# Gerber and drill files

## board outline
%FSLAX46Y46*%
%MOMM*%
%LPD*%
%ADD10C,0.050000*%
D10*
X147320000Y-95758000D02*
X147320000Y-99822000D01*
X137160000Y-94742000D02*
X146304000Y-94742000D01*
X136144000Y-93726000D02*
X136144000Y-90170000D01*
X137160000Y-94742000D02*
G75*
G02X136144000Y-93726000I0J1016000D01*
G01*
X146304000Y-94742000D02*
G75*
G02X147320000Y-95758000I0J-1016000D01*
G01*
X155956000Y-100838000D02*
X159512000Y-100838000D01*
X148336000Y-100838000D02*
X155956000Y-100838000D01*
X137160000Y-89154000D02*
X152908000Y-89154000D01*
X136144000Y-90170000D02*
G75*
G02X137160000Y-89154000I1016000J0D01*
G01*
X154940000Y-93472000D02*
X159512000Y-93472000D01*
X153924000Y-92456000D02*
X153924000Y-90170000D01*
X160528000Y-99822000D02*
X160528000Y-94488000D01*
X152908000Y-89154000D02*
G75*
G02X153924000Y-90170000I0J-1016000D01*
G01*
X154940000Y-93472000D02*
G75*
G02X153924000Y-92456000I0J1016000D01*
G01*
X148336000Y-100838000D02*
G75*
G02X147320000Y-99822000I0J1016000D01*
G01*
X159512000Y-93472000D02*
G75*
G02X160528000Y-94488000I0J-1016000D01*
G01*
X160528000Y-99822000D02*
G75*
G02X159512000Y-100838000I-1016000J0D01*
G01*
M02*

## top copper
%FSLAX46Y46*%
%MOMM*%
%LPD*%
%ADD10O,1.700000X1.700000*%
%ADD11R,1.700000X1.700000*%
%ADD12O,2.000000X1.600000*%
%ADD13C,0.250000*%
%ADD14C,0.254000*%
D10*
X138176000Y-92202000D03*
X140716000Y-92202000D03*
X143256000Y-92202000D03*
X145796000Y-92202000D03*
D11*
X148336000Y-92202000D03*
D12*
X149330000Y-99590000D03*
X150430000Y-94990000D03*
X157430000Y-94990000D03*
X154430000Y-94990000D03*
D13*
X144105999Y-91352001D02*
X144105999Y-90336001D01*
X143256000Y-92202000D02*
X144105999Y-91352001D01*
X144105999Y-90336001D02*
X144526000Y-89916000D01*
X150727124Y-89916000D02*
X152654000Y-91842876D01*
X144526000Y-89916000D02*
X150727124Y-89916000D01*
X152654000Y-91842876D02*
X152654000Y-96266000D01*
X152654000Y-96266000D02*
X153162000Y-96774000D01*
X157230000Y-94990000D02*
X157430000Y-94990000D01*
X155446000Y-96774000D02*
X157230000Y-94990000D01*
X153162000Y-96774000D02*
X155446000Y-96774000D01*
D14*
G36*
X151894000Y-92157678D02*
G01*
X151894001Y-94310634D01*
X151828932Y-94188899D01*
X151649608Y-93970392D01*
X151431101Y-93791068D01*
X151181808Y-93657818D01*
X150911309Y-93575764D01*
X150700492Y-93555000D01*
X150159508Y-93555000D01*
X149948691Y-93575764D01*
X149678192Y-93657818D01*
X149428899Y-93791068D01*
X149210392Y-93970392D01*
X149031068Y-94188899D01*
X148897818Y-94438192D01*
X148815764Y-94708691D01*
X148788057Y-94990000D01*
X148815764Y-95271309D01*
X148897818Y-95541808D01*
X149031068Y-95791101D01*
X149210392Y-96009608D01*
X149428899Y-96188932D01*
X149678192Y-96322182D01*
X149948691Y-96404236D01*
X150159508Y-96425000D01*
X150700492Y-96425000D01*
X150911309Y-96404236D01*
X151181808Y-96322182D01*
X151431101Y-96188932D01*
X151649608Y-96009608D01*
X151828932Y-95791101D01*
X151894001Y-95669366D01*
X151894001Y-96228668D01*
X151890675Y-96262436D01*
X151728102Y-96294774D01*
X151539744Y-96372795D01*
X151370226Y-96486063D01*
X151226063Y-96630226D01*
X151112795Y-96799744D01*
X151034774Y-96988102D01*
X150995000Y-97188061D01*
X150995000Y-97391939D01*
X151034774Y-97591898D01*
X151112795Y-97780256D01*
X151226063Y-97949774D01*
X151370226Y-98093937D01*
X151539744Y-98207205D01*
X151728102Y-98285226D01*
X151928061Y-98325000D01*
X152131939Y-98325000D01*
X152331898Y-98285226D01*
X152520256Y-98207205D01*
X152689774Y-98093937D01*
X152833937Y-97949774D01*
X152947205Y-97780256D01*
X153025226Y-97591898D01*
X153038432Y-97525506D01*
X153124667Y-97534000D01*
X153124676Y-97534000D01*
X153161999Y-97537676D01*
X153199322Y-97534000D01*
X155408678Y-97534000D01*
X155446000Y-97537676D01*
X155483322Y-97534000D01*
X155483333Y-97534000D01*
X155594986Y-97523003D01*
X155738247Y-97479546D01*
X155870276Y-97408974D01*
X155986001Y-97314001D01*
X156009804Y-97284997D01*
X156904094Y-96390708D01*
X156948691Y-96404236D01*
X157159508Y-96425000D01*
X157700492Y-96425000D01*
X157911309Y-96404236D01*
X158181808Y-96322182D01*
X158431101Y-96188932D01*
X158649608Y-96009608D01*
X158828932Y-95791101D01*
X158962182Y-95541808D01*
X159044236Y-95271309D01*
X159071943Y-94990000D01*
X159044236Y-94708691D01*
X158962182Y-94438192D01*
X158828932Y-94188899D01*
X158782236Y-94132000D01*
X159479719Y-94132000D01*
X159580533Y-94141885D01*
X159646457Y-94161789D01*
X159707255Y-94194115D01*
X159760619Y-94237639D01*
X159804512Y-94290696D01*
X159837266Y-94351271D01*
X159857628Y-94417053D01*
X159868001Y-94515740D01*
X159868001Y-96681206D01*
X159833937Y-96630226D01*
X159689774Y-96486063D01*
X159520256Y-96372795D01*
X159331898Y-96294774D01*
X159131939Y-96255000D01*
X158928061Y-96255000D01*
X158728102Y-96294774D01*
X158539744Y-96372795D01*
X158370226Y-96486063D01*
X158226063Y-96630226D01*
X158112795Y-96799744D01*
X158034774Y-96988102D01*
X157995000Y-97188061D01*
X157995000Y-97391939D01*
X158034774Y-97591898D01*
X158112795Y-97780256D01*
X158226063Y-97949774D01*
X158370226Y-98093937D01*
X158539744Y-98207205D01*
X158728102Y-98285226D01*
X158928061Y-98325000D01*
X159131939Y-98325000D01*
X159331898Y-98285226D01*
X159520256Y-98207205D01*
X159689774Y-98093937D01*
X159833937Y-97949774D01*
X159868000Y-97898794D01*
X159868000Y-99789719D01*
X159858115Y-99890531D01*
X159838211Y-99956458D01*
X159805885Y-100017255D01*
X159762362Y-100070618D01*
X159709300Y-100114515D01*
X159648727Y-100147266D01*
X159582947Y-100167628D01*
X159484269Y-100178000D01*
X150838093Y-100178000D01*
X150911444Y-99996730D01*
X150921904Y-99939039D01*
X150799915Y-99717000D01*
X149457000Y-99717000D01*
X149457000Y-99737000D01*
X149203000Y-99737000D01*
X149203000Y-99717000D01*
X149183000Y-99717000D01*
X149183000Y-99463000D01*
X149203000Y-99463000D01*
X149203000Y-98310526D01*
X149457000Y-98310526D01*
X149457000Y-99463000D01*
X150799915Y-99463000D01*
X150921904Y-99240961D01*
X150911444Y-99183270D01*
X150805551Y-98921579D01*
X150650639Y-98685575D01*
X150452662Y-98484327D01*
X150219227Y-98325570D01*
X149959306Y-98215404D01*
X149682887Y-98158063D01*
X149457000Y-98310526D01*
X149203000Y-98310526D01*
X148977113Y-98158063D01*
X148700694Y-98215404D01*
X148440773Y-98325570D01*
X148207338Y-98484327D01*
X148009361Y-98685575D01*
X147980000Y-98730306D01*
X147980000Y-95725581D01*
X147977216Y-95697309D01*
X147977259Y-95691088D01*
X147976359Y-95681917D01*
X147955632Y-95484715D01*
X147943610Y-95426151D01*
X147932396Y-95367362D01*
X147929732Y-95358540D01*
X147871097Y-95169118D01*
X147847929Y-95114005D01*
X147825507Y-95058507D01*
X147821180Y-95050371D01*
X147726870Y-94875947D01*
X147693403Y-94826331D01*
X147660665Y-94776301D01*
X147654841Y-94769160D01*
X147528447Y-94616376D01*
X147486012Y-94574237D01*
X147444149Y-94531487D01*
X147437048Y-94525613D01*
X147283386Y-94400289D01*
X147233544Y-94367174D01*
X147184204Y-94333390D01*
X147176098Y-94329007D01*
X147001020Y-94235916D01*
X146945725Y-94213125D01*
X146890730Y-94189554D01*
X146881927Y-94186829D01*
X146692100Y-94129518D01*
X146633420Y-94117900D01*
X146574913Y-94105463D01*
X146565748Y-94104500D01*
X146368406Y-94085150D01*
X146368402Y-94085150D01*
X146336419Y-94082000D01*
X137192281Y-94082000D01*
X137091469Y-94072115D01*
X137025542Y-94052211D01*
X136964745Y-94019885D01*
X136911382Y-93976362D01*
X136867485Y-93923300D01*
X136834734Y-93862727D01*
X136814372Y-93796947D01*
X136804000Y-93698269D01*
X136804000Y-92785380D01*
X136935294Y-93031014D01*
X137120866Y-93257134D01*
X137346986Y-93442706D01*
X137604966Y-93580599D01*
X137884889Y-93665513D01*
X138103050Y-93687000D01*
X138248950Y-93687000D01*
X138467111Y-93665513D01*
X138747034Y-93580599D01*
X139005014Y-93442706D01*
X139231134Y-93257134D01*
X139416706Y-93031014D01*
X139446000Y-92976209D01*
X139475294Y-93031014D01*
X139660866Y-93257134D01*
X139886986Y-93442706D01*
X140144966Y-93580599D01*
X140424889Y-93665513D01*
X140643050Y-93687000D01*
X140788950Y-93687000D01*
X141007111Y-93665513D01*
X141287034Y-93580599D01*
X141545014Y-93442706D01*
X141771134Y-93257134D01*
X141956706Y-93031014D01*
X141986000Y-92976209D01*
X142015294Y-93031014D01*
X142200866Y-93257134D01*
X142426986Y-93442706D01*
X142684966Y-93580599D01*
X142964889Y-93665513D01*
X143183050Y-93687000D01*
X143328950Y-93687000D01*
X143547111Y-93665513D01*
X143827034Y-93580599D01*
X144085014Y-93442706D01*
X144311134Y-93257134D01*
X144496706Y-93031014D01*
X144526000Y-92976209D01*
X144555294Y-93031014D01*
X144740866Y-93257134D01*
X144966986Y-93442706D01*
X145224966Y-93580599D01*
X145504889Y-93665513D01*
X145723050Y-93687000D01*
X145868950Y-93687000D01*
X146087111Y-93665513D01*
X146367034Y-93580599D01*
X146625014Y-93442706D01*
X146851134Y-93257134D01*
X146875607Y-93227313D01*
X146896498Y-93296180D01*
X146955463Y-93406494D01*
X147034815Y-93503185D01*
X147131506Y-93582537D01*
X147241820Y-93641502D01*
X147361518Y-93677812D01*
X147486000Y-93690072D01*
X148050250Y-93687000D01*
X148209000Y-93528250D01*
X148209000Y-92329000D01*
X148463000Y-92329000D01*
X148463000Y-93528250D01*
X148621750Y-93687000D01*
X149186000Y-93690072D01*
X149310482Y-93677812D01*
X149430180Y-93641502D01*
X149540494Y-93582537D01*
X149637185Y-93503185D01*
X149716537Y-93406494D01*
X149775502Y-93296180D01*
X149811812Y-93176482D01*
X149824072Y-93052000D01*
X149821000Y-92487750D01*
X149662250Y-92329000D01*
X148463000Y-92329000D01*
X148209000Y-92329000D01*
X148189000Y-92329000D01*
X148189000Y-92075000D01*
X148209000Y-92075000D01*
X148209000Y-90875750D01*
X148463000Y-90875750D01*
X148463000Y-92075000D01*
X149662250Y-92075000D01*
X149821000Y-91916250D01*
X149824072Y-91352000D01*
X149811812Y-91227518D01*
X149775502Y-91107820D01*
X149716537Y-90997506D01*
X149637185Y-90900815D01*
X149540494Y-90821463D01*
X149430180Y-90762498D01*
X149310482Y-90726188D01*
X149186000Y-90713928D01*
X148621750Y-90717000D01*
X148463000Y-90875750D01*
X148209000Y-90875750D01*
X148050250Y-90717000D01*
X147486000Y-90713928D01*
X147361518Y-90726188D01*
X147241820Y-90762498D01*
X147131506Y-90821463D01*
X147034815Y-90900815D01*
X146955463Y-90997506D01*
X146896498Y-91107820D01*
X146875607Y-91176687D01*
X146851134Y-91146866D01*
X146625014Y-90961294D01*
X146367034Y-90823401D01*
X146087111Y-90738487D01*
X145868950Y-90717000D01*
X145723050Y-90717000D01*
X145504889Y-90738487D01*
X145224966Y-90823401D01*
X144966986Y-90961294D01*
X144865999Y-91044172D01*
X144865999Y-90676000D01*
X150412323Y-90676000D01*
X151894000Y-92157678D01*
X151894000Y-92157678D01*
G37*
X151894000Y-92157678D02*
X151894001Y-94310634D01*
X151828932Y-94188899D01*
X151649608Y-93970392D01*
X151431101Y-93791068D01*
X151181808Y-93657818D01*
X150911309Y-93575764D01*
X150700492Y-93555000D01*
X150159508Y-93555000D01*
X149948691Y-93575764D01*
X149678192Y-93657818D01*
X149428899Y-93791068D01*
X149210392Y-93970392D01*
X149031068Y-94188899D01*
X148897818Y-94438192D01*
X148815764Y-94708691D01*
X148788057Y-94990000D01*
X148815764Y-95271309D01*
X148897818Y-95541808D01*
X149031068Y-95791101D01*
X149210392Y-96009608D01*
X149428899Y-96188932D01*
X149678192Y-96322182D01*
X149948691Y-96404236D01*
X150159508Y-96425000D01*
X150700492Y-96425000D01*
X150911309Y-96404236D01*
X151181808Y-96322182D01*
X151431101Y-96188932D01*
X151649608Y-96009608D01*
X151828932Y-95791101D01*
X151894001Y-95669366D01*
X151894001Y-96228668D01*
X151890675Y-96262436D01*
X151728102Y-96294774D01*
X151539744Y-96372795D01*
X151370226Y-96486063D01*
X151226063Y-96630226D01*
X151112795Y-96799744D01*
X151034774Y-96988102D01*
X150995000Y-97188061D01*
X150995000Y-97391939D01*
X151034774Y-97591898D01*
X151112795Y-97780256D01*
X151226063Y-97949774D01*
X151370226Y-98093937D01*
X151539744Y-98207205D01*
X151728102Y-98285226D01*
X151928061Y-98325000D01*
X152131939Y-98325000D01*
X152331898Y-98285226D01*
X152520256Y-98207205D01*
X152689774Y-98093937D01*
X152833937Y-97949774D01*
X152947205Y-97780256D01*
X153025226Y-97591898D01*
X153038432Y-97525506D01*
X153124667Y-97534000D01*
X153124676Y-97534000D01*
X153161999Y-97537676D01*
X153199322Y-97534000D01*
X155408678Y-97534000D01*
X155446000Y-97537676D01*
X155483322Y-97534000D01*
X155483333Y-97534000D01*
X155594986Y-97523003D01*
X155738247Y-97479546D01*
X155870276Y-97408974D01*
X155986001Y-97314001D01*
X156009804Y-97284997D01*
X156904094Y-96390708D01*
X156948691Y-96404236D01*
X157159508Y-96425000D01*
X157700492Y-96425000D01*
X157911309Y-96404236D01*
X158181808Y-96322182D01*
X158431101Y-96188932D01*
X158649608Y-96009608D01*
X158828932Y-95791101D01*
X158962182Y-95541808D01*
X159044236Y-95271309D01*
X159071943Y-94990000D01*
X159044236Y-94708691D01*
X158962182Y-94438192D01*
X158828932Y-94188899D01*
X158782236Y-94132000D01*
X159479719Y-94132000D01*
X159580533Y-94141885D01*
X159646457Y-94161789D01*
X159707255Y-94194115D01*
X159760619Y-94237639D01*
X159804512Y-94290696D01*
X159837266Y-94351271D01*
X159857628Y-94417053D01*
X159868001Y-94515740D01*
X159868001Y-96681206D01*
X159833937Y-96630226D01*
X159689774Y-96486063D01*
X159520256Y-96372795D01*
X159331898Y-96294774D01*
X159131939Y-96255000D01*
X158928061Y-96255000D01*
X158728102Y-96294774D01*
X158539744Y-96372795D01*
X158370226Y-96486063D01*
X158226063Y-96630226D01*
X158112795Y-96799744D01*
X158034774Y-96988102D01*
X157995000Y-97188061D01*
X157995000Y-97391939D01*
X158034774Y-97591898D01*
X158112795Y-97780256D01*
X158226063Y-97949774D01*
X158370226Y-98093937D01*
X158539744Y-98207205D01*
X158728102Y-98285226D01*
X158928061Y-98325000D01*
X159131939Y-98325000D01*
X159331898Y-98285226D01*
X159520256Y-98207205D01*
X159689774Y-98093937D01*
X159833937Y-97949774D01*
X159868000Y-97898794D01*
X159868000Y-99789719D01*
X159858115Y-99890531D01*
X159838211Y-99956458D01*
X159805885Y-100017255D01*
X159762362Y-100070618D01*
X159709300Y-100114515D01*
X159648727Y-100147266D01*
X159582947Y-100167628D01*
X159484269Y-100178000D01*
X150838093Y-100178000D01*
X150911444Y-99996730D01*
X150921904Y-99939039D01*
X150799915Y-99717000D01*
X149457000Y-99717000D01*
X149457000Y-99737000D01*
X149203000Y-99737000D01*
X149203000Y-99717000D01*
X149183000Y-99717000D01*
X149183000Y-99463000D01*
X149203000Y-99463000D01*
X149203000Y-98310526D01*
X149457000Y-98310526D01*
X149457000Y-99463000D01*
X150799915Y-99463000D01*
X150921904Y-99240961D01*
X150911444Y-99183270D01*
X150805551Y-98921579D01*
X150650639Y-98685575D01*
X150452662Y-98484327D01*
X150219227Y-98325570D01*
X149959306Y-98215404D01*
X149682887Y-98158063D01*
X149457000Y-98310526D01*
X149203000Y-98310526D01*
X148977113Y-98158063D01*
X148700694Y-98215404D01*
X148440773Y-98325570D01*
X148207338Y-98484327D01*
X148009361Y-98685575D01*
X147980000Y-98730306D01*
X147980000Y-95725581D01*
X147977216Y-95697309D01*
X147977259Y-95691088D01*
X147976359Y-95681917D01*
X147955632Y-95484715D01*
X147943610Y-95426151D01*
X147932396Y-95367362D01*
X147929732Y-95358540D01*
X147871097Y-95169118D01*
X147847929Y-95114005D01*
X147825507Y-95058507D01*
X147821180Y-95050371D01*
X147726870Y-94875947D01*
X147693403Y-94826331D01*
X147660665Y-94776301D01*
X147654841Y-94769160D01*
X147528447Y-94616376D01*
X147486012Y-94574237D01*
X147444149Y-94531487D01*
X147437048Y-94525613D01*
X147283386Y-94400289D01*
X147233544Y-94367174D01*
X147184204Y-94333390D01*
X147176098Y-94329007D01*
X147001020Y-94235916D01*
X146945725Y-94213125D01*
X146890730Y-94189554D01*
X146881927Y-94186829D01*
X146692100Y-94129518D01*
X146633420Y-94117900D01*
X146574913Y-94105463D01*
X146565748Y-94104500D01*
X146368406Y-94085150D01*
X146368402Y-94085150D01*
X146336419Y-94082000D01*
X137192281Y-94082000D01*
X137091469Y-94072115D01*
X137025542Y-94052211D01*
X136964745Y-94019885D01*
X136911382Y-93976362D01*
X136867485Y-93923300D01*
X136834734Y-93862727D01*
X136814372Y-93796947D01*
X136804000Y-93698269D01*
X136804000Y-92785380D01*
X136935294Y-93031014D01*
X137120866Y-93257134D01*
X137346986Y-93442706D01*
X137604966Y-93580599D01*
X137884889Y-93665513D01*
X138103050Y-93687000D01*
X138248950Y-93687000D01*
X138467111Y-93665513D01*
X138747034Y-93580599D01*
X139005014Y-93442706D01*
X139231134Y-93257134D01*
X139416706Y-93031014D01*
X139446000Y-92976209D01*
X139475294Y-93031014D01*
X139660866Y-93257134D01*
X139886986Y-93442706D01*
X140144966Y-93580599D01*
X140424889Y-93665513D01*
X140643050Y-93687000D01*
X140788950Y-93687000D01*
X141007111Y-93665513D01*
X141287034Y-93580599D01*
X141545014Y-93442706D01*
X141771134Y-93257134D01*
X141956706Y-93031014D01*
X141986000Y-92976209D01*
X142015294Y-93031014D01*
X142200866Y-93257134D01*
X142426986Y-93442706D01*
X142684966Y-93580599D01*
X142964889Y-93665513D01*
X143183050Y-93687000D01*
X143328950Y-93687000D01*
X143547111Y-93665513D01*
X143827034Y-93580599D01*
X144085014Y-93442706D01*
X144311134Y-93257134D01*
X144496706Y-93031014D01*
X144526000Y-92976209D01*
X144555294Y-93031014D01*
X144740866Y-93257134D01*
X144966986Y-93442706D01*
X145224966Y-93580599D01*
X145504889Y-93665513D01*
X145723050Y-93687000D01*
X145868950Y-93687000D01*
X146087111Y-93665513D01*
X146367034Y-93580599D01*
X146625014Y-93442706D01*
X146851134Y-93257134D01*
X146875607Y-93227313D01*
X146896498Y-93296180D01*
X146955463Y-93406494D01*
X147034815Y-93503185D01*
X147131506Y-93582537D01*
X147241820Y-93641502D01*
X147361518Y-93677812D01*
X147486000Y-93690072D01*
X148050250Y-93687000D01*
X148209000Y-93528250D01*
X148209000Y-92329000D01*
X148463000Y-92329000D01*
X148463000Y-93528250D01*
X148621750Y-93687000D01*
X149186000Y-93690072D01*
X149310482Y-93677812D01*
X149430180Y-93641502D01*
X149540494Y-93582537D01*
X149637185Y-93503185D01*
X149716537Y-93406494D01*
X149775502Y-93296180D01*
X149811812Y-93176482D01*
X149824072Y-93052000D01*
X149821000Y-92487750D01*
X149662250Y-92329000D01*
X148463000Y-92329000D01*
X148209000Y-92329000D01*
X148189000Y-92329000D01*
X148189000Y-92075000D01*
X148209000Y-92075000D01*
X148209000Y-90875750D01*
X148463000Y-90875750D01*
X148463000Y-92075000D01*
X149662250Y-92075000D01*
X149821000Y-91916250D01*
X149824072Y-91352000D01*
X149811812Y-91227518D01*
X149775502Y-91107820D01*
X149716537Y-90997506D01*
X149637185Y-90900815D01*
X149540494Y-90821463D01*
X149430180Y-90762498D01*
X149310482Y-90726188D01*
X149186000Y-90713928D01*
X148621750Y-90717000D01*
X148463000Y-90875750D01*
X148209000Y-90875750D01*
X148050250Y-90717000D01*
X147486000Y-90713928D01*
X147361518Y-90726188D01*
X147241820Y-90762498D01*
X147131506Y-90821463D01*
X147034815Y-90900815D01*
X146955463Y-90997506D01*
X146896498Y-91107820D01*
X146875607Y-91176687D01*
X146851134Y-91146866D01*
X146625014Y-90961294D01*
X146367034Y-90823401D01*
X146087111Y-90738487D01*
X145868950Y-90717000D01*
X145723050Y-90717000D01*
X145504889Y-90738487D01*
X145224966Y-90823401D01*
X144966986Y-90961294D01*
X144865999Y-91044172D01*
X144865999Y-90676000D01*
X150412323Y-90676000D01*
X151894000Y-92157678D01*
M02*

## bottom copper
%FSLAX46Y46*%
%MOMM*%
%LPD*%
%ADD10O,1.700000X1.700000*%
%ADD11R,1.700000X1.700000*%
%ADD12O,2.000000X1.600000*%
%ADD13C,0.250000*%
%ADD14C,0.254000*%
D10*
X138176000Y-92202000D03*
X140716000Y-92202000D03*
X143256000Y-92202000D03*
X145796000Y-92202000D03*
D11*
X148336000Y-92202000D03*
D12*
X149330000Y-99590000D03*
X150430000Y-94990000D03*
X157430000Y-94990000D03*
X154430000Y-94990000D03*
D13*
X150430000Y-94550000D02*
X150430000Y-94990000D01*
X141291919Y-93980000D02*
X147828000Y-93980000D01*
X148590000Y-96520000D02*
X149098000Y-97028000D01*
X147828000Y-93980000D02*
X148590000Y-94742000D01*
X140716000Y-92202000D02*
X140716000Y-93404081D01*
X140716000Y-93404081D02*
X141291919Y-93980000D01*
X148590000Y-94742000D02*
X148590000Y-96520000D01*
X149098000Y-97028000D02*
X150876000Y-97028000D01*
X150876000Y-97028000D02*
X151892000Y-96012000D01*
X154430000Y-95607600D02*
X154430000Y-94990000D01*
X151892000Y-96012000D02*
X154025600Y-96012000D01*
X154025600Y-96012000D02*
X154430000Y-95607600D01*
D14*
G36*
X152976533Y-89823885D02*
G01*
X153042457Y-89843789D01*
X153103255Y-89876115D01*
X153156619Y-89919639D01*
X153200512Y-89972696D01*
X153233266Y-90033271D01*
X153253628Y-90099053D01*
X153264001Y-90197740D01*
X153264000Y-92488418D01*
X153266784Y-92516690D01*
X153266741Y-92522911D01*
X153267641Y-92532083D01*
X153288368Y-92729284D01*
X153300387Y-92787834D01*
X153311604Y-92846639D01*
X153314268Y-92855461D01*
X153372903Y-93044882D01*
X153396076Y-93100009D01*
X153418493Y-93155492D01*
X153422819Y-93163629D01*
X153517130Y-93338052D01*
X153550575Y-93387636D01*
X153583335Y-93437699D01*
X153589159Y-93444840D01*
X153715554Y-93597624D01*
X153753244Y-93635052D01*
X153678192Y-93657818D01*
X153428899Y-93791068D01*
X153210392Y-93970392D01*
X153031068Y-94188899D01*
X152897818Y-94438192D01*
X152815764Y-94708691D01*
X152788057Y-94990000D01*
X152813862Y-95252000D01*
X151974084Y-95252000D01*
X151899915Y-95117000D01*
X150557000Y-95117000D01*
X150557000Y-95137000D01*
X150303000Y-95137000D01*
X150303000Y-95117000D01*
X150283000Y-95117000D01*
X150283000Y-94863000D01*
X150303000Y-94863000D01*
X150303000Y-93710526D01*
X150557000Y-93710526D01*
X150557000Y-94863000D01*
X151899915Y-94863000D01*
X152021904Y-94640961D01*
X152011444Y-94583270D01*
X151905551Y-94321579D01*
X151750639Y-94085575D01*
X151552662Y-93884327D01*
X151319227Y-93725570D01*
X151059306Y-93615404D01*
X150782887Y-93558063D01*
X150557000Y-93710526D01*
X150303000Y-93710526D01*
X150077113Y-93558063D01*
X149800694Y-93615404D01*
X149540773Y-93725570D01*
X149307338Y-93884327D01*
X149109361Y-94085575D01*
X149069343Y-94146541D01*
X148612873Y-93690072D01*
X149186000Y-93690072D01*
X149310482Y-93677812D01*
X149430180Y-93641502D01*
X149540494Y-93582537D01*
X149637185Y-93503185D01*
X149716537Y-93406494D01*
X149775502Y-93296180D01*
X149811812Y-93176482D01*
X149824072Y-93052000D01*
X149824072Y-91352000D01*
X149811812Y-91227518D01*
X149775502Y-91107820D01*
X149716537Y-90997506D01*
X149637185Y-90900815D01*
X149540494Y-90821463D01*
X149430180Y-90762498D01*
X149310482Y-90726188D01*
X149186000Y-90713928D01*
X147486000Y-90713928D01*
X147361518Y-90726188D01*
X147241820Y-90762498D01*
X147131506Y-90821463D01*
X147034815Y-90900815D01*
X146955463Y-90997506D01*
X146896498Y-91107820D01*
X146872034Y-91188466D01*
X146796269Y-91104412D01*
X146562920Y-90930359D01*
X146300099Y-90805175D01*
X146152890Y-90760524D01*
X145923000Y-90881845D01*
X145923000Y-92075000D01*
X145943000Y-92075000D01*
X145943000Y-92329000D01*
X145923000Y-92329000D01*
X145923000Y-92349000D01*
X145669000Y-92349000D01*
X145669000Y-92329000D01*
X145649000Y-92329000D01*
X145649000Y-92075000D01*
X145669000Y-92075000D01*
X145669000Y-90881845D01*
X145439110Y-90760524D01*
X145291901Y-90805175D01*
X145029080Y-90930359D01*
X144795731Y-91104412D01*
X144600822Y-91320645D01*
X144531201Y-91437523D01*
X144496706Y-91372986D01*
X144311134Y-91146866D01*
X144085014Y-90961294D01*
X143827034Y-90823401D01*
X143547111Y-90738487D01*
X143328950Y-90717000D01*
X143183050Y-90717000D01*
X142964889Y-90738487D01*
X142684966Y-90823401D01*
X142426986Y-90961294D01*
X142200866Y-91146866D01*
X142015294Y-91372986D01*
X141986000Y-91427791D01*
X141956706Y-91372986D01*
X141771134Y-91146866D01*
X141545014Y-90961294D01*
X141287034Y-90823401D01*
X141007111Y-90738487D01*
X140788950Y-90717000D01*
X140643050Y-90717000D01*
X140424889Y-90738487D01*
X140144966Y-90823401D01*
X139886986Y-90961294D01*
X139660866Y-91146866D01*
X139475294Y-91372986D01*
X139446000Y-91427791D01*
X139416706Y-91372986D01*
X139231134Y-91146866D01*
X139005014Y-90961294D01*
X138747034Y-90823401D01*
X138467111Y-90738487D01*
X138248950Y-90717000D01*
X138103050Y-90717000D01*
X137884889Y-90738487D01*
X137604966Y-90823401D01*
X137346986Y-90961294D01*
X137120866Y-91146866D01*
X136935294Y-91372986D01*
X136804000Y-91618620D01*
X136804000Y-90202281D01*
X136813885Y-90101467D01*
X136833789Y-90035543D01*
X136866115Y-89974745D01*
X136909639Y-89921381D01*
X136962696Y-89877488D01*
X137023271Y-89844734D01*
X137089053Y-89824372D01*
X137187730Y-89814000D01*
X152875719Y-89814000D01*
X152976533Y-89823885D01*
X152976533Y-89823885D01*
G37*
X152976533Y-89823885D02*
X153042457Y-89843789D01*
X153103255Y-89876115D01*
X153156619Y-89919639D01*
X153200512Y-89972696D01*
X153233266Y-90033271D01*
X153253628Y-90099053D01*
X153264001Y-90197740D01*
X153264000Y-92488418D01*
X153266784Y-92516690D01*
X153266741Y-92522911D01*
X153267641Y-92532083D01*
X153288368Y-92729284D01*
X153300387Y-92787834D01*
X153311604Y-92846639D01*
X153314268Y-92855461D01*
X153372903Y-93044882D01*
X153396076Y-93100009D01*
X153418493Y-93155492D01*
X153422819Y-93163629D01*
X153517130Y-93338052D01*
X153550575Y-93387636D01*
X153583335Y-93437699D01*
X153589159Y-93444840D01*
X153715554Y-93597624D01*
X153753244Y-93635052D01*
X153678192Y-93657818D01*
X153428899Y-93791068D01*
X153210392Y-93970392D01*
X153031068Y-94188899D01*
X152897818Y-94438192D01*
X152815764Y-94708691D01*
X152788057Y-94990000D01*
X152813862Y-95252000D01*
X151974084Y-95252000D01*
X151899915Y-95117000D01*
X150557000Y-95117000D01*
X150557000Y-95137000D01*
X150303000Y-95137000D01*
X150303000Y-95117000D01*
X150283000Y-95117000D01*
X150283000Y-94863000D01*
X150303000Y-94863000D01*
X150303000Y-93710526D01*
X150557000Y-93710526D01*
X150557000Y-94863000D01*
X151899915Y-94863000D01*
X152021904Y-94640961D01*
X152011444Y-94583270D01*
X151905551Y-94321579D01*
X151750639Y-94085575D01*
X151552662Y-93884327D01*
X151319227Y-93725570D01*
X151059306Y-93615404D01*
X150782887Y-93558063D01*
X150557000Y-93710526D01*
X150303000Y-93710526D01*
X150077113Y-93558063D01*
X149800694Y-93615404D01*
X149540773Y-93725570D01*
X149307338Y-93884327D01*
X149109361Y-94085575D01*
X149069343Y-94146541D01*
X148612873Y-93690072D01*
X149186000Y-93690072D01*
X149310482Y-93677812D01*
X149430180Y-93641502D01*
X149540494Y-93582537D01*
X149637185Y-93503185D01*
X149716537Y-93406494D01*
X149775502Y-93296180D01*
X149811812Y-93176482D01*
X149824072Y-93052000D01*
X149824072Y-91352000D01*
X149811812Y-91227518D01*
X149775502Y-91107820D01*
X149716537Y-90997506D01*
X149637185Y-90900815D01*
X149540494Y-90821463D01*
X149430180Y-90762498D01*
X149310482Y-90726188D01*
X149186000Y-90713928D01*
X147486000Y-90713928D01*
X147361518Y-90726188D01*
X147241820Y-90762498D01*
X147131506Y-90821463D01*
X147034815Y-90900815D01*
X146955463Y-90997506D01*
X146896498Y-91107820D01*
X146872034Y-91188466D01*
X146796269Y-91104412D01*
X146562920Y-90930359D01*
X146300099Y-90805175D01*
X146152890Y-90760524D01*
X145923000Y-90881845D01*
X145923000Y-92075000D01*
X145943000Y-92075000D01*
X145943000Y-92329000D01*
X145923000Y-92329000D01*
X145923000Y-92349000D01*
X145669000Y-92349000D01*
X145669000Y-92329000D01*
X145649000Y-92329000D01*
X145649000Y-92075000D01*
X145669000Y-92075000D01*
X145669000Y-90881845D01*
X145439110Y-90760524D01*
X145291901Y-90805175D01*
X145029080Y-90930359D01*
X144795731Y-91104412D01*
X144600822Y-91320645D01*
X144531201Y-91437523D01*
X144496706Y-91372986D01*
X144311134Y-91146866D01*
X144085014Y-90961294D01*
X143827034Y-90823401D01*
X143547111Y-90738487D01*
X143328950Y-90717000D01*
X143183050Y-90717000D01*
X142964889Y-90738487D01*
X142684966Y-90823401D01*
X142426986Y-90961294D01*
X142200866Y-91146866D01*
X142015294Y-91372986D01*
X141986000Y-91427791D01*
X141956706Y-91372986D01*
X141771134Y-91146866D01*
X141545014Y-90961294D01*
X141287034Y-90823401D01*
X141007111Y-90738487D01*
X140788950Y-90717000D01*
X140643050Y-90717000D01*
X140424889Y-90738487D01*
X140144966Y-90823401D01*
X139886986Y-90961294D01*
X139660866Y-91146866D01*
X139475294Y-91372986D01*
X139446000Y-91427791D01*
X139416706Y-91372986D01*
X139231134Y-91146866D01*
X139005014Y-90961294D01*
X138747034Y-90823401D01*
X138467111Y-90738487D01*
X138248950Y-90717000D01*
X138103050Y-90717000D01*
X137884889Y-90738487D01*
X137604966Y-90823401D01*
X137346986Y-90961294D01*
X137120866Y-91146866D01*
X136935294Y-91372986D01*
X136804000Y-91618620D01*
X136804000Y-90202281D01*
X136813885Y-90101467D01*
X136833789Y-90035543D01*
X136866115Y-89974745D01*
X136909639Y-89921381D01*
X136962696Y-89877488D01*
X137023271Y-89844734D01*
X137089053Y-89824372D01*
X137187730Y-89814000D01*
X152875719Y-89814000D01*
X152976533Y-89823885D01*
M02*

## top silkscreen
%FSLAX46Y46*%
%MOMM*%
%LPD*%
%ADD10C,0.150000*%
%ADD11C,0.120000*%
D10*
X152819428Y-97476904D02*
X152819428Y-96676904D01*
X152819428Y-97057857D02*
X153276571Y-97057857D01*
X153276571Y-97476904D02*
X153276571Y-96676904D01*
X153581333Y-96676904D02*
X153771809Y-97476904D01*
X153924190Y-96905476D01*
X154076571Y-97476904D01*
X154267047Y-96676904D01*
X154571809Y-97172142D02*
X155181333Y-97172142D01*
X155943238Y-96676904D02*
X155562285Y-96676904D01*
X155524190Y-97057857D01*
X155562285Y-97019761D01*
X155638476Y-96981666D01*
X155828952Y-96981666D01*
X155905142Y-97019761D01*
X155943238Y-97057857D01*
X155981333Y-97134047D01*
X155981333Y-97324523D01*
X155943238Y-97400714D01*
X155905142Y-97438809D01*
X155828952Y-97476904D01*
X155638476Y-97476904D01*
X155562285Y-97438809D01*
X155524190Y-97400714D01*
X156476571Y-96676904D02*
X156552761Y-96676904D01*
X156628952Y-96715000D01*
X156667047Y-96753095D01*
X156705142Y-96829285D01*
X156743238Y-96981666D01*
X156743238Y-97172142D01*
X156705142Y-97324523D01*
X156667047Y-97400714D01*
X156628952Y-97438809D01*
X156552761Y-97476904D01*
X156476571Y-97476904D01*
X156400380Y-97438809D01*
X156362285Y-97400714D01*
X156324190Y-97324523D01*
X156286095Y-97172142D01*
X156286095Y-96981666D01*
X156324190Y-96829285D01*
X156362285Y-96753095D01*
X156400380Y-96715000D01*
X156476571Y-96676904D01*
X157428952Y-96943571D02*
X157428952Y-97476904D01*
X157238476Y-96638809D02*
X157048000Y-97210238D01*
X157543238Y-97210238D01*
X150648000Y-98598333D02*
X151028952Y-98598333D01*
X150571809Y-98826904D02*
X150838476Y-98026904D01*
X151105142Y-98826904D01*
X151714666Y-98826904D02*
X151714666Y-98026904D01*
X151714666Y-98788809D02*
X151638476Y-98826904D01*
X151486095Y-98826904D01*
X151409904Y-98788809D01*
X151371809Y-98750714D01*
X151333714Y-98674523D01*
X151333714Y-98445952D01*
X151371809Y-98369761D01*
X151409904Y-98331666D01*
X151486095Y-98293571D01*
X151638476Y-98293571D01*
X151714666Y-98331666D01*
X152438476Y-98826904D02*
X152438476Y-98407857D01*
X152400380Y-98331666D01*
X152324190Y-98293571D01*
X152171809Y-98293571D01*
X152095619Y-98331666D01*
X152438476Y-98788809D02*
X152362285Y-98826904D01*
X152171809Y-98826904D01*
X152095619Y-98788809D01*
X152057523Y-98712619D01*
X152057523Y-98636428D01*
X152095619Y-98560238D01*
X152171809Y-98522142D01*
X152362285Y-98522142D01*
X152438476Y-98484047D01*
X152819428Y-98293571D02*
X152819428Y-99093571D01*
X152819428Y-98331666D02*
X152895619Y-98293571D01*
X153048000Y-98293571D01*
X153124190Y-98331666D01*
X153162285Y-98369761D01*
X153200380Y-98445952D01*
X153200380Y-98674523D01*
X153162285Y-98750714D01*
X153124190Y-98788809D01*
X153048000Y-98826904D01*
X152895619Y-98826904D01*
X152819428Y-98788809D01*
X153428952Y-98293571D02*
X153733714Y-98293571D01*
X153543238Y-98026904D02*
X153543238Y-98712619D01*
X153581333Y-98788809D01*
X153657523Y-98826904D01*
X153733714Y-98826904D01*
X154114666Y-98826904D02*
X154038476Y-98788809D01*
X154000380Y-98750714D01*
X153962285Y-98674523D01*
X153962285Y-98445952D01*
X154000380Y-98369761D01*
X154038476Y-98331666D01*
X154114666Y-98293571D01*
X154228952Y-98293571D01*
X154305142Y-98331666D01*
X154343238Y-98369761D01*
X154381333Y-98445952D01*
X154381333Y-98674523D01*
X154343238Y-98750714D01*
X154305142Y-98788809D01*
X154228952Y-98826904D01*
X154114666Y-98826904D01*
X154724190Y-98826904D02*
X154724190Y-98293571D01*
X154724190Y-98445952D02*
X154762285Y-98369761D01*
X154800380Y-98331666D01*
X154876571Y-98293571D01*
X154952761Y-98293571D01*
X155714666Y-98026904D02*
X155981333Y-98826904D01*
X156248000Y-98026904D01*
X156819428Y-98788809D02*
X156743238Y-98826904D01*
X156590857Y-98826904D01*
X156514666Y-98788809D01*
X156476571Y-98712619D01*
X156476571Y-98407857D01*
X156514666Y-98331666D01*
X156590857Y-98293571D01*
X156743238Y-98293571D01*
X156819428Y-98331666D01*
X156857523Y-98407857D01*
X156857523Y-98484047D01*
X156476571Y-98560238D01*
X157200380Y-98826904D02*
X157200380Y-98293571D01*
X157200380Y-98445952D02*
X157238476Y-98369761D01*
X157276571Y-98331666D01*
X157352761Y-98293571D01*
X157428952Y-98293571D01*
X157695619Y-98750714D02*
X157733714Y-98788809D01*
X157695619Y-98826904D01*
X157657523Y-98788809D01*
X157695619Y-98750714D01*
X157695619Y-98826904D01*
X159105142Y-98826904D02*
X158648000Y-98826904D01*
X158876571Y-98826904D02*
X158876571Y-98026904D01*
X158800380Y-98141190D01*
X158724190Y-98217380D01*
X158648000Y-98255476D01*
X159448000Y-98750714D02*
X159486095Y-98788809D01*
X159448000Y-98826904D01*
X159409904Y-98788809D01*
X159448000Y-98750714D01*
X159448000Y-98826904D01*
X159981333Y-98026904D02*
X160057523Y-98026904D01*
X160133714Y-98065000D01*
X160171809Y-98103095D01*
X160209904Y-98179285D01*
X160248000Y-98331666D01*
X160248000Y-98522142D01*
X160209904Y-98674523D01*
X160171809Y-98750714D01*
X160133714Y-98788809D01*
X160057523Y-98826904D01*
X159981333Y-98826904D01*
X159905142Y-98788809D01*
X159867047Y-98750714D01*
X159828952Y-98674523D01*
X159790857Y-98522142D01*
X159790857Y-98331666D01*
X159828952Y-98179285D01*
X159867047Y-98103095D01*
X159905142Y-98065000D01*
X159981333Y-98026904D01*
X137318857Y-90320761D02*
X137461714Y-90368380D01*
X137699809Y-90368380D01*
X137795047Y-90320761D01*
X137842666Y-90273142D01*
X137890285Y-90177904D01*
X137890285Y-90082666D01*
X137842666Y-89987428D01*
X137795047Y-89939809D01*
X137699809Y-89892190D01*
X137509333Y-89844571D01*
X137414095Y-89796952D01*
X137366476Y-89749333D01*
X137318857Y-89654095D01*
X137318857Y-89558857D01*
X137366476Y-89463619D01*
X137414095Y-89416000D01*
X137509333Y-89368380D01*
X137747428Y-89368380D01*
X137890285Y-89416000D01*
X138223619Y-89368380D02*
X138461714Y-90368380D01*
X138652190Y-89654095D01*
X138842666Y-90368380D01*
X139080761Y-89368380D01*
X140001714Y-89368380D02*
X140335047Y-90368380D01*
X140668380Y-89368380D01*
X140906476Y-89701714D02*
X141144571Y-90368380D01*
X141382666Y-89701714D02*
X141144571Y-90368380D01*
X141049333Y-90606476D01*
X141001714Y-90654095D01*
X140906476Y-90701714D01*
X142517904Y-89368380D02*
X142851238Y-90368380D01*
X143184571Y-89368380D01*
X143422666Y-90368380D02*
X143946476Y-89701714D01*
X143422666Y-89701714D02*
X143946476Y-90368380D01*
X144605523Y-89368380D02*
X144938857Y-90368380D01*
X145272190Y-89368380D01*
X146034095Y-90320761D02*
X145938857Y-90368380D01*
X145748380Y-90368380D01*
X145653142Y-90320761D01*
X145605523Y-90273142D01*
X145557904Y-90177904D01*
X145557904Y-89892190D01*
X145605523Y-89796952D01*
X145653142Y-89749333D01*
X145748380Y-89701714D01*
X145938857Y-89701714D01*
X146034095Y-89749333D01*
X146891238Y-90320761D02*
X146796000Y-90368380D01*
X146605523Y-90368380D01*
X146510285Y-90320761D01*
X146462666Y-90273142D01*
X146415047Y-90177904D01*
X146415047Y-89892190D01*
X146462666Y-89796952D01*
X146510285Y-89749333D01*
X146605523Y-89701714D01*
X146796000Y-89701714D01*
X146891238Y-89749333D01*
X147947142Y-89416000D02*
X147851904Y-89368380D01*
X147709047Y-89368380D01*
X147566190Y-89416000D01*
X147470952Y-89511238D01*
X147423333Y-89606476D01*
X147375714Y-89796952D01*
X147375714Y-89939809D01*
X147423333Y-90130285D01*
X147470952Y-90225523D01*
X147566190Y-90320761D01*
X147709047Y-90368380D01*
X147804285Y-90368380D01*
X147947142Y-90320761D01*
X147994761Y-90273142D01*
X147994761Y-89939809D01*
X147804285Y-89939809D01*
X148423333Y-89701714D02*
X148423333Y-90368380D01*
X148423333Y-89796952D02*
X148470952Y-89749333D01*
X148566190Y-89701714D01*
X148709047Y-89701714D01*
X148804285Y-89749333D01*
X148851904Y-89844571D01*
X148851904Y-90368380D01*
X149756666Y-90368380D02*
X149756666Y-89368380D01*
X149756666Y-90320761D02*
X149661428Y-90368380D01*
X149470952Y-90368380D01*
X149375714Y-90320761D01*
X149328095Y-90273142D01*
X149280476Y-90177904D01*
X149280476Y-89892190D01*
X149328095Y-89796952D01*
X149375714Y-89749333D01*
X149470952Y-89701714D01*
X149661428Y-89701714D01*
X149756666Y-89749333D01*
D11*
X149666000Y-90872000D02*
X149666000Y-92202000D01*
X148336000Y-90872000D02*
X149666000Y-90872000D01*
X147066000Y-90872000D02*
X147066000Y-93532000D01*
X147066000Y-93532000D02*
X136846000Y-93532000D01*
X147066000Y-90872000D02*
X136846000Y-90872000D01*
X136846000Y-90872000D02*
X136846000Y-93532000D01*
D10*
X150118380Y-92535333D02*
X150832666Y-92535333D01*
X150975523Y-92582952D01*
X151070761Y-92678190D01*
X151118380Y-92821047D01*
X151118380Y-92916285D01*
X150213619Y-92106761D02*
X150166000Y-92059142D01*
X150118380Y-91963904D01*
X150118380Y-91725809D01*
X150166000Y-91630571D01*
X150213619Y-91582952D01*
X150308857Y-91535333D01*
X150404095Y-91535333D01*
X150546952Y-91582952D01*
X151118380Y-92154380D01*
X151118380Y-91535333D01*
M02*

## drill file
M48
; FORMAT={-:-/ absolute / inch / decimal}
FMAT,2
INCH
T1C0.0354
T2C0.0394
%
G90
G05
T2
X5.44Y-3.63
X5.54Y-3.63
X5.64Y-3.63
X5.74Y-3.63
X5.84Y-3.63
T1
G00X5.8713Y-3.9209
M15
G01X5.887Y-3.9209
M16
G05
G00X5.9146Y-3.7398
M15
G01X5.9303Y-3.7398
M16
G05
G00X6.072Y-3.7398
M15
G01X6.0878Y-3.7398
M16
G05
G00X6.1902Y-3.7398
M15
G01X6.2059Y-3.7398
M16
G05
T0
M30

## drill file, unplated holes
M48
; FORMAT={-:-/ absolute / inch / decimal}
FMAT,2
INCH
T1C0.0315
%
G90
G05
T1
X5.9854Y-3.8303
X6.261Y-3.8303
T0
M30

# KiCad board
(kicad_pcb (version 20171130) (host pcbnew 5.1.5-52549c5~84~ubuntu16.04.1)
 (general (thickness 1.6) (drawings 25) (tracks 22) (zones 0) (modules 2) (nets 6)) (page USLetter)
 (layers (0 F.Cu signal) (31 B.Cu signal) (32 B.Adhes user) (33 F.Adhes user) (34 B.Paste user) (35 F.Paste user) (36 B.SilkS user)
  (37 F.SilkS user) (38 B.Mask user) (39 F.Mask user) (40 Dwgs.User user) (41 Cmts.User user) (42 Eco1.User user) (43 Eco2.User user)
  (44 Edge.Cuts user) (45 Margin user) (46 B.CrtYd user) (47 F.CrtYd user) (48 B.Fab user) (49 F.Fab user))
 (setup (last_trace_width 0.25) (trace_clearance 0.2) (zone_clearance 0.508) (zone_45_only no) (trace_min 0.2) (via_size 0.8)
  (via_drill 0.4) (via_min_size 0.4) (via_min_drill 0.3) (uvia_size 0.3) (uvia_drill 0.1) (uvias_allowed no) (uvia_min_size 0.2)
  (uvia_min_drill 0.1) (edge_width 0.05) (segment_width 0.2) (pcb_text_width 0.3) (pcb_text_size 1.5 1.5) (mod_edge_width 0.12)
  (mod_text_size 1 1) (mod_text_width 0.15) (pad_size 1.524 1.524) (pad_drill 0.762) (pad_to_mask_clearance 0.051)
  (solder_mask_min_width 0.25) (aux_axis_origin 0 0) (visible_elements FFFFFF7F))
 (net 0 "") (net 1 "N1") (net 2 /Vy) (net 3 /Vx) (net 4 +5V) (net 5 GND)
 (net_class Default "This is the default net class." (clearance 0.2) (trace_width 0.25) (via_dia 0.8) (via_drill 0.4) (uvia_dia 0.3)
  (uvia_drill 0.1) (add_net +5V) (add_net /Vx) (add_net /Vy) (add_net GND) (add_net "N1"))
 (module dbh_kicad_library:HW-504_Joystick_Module (layer F.Cu) (at 148.336 92.202 270)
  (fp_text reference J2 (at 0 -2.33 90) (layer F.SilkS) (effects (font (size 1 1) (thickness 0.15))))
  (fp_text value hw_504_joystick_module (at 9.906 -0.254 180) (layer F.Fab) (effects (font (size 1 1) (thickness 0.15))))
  (fp_line (start -1.33 -1.33) (end 0 -1.33) (layer F.SilkS) (width 0.12))
  (fp_line (start -1.33 0) (end -1.33 -1.33) (layer F.SilkS) (width 0.12))
  (fp_line (start -1.33 1.27) (end 1.33 1.27) (layer F.SilkS) (width 0.12))
  (fp_line (start 1.33 1.27) (end 1.33 11.49) (layer F.SilkS) (width 0.12))
  (fp_line (start -1.33 1.27) (end -1.33 11.49) (layer F.SilkS) (width 0.12))
  (fp_line (start -1.33 11.49) (end 1.33 11.49) (layer F.SilkS) (width 0.12))
  (pad 5 thru_hole oval (at 0 10.16 270) (size 1.7 1.7) (drill 1) (layers *.Cu *.Mask) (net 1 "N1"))
  (pad 4 thru_hole oval (at 0 7.62 270) (size 1.7 1.7) (drill 1) (layers *.Cu *.Mask) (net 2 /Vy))
  (pad 3 thru_hole oval (at 0 5.08 270) (size 1.7 1.7) (drill 1) (layers *.Cu *.Mask) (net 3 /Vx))
  (pad 2 thru_hole oval (at 0 2.54 270) (size 1.7 1.7) (drill 1) (layers *.Cu *.Mask) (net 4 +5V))
  (pad 1 thru_hole rect (at 0 0 270) (size 1.7 1.7) (drill 1) (layers *.Cu *.Mask) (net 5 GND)))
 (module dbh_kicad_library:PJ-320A (layer B.Cu) (at 157.48 95.25 180)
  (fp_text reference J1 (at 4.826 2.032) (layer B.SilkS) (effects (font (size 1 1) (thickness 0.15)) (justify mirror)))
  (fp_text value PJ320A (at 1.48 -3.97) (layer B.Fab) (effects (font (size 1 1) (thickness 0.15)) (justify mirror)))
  (pad 5 thru_hole oval (at 8.15 -4.34 90) (size 1.6 2) (drill oval 0.9 1.3) (layers *.Cu *.Mask) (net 5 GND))
  (pad 4 thru_hole oval (at 7.05 0.26 90) (size 1.6 2) (drill oval 0.9 1.3) (layers *.Cu *.Mask) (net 4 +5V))
  (pad 2 thru_hole oval (at 0.05 0.26 90) (size 1.6 2) (drill oval 0.9 1.3) (layers *.Cu *.Mask) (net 3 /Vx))
  (pad "" np_thru_hole circle (at 5.45 -2.04 90) (size 0.8 0.8) (drill 0.8) (layers *.Cu *.Mask))
  (pad "" np_thru_hole circle (at -1.55 -2.04 90) (size 0.8 0.8) (drill 0.8) (layers *.Cu *.Mask))
  (pad 3 thru_hole oval (at 3.05 0.26 90) (size 1.6 2) (drill oval 0.9 1.3) (layers *.Cu *.Mask) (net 2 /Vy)))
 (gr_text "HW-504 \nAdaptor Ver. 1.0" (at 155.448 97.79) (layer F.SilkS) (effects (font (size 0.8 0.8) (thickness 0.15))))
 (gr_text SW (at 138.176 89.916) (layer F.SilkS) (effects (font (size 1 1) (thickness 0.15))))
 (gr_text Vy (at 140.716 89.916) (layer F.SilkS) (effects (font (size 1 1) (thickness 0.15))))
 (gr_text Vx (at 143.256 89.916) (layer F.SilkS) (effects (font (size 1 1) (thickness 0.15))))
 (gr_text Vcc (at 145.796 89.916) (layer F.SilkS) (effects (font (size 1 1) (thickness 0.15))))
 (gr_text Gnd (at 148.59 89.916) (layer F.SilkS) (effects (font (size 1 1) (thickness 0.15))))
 (gr_line (start 147.32 95.758) (end 147.32 99.822) (layer Edge.Cuts) (width 0.05))
 (gr_line (start 137.16 94.742) (end 146.304 94.742) (layer Edge.Cuts) (width 0.05))
 (gr_line (start 136.144 93.726) (end 136.144 90.17) (layer Edge.Cuts) (width 0.05))
 (gr_arc (start 137.16 93.726) (end 136.144 93.726) (angle -90) (layer Edge.Cuts) (width 0.05))
 (gr_arc (start 146.304 95.758) (end 147.32 95.758) (angle -90) (layer Edge.Cuts) (width 0.05))
 (gr_line (start 155.956 100.838) (end 159.512 100.838) (layer Edge.Cuts) (width 0.05))
 (gr_line (start 148.336 100.838) (end 155.956 100.838) (layer Edge.Cuts) (width 0.05))
 (gr_line (start 137.16 89.154) (end 152.908 89.154) (layer Edge.Cuts) (width 0.05))
 (gr_arc (start 137.16 90.17) (end 137.16 89.154) (angle -90) (layer Edge.Cuts) (width 0.05))
 (gr_line (start 154.94 93.472) (end 159.512 93.472) (layer Edge.Cuts) (width 0.05))
 (gr_line (start 153.924 92.456) (end 153.924 90.17) (layer Edge.Cuts) (width 0.05))
 (gr_line (start 160.528 99.822) (end 160.528 94.488) (layer Edge.Cuts) (width 0.05))
 (gr_arc (start 152.908 90.17) (end 153.924 90.17) (angle -90) (layer Edge.Cuts) (width 0.05))
 (gr_arc (start 154.94 92.456) (end 153.924 92.456) (angle -90) (layer Edge.Cuts) (width 0.05))
 (gr_arc (start 148.336 99.822) (end 147.32 99.822) (angle -90) (layer Edge.Cuts) (width 0.05))
 (gr_arc (start 159.512 94.488) (end 160.528 94.488) (angle -90) (layer Edge.Cuts) (width 0.05))
 (gr_arc (start 159.512 99.822) (end 159.512 100.838) (angle -90) (layer Edge.Cuts) (width 0.05))
 (segment (start 150.43 94.55) (end 150.43 94.99) (width 0.25) (layer B.Cu) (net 4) (status 30))
 (segment (start 144.105999 91.352001) (end 144.105999 90.336001) (width 0.25) (layer F.Cu) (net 3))
 (segment (start 143.256 92.202) (end 144.105999 91.352001) (width 0.25) (layer F.Cu) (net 3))
 (segment (start 144.105999 90.336001) (end 144.526 89.916) (width 0.25) (layer F.Cu) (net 3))
 (segment (start 150.727124 89.916) (end 152.654 91.842876) (width 0.25) (layer F.Cu) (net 3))
 (segment (start 144.526 89.916) (end 150.727124 89.916) (width 0.25) (layer F.Cu) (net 3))
 (segment (start 152.654 91.842876) (end 152.654 96.266) (width 0.25) (layer F.Cu) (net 3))
 (segment (start 152.654 96.266) (end 153.162 96.774) (width 0.25) (layer F.Cu) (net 3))
 (segment (start 157.23 94.99) (end 157.43 94.99) (width 0.25) (layer F.Cu) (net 3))
 (segment (start 155.446 96.774) (end 157.23 94.99) (width 0.25) (layer F.Cu) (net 3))
 (segment (start 153.162 96.774) (end 155.446 96.774) (width 0.25) (layer F.Cu) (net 3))
 (segment (start 141.291919 93.98) (end 147.828 93.98) (width 0.25) (layer B.Cu) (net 2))
 (segment (start 148.59 96.52) (end 149.098 97.028) (width 0.25) (layer B.Cu) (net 2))
 (segment (start 147.828 93.98) (end 148.59 94.742) (width 0.25) (layer B.Cu) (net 2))
 (segment (start 140.716 92.202) (end 140.716 93.404081) (width 0.25) (layer B.Cu) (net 2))
 (segment (start 140.716 93.404081) (end 141.291919 93.98) (width 0.25) (layer B.Cu) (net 2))
 (segment (start 148.59 94.742) (end 148.59 96.52) (width 0.25) (layer B.Cu) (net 2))
 (segment (start 149.098 97.028) (end 150.876 97.028) (width 0.25) (layer B.Cu) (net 2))
 (segment (start 150.876 97.028) (end 151.892 96.012) (width 0.25) (layer B.Cu) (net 2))
 (segment (start 154.43 95.6076) (end 154.43 94.99) (width 0.25) (layer B.Cu) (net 2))
 (segment (start 151.892 96.012) (end 154.0256 96.012) (width 0.25) (layer B.Cu) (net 2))
 (segment (start 154.0256 96.012) (end 154.43 95.6076) (width 0.25) (layer B.Cu) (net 2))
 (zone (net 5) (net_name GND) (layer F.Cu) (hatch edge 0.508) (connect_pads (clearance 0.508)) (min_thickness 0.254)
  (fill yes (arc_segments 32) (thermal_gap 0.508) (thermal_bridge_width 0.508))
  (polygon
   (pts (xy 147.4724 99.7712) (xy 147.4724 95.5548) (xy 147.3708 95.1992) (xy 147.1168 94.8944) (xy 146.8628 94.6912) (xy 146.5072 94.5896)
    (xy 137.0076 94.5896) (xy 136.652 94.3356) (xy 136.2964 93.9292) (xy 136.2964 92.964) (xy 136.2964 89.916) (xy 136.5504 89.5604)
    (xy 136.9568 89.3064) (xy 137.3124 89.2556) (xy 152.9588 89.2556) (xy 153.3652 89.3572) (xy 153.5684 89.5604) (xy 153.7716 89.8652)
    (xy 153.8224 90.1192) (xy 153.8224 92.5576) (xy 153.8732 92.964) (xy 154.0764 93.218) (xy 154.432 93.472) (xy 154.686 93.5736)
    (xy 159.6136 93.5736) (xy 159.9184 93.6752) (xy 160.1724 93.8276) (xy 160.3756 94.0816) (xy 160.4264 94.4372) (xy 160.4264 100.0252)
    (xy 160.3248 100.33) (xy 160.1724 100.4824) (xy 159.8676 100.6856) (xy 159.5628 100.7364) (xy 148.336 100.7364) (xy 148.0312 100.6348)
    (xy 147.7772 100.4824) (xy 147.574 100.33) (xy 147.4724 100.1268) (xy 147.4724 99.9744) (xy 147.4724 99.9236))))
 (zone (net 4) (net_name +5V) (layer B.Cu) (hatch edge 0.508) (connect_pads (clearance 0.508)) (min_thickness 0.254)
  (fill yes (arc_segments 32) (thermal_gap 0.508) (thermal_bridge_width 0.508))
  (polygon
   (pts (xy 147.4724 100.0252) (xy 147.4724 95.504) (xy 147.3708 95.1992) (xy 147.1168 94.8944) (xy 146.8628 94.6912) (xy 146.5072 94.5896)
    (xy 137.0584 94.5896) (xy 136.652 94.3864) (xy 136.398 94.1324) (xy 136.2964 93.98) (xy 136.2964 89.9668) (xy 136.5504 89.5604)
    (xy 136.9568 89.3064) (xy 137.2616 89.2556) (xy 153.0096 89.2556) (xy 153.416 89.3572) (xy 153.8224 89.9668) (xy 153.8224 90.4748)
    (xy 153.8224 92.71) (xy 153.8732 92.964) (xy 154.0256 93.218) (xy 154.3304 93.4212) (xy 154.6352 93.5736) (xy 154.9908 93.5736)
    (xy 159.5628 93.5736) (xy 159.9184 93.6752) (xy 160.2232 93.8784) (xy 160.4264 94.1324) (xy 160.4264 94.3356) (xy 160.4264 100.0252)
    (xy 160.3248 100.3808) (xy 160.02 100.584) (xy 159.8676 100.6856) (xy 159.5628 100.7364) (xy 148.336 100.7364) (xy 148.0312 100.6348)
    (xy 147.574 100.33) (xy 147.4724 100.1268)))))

